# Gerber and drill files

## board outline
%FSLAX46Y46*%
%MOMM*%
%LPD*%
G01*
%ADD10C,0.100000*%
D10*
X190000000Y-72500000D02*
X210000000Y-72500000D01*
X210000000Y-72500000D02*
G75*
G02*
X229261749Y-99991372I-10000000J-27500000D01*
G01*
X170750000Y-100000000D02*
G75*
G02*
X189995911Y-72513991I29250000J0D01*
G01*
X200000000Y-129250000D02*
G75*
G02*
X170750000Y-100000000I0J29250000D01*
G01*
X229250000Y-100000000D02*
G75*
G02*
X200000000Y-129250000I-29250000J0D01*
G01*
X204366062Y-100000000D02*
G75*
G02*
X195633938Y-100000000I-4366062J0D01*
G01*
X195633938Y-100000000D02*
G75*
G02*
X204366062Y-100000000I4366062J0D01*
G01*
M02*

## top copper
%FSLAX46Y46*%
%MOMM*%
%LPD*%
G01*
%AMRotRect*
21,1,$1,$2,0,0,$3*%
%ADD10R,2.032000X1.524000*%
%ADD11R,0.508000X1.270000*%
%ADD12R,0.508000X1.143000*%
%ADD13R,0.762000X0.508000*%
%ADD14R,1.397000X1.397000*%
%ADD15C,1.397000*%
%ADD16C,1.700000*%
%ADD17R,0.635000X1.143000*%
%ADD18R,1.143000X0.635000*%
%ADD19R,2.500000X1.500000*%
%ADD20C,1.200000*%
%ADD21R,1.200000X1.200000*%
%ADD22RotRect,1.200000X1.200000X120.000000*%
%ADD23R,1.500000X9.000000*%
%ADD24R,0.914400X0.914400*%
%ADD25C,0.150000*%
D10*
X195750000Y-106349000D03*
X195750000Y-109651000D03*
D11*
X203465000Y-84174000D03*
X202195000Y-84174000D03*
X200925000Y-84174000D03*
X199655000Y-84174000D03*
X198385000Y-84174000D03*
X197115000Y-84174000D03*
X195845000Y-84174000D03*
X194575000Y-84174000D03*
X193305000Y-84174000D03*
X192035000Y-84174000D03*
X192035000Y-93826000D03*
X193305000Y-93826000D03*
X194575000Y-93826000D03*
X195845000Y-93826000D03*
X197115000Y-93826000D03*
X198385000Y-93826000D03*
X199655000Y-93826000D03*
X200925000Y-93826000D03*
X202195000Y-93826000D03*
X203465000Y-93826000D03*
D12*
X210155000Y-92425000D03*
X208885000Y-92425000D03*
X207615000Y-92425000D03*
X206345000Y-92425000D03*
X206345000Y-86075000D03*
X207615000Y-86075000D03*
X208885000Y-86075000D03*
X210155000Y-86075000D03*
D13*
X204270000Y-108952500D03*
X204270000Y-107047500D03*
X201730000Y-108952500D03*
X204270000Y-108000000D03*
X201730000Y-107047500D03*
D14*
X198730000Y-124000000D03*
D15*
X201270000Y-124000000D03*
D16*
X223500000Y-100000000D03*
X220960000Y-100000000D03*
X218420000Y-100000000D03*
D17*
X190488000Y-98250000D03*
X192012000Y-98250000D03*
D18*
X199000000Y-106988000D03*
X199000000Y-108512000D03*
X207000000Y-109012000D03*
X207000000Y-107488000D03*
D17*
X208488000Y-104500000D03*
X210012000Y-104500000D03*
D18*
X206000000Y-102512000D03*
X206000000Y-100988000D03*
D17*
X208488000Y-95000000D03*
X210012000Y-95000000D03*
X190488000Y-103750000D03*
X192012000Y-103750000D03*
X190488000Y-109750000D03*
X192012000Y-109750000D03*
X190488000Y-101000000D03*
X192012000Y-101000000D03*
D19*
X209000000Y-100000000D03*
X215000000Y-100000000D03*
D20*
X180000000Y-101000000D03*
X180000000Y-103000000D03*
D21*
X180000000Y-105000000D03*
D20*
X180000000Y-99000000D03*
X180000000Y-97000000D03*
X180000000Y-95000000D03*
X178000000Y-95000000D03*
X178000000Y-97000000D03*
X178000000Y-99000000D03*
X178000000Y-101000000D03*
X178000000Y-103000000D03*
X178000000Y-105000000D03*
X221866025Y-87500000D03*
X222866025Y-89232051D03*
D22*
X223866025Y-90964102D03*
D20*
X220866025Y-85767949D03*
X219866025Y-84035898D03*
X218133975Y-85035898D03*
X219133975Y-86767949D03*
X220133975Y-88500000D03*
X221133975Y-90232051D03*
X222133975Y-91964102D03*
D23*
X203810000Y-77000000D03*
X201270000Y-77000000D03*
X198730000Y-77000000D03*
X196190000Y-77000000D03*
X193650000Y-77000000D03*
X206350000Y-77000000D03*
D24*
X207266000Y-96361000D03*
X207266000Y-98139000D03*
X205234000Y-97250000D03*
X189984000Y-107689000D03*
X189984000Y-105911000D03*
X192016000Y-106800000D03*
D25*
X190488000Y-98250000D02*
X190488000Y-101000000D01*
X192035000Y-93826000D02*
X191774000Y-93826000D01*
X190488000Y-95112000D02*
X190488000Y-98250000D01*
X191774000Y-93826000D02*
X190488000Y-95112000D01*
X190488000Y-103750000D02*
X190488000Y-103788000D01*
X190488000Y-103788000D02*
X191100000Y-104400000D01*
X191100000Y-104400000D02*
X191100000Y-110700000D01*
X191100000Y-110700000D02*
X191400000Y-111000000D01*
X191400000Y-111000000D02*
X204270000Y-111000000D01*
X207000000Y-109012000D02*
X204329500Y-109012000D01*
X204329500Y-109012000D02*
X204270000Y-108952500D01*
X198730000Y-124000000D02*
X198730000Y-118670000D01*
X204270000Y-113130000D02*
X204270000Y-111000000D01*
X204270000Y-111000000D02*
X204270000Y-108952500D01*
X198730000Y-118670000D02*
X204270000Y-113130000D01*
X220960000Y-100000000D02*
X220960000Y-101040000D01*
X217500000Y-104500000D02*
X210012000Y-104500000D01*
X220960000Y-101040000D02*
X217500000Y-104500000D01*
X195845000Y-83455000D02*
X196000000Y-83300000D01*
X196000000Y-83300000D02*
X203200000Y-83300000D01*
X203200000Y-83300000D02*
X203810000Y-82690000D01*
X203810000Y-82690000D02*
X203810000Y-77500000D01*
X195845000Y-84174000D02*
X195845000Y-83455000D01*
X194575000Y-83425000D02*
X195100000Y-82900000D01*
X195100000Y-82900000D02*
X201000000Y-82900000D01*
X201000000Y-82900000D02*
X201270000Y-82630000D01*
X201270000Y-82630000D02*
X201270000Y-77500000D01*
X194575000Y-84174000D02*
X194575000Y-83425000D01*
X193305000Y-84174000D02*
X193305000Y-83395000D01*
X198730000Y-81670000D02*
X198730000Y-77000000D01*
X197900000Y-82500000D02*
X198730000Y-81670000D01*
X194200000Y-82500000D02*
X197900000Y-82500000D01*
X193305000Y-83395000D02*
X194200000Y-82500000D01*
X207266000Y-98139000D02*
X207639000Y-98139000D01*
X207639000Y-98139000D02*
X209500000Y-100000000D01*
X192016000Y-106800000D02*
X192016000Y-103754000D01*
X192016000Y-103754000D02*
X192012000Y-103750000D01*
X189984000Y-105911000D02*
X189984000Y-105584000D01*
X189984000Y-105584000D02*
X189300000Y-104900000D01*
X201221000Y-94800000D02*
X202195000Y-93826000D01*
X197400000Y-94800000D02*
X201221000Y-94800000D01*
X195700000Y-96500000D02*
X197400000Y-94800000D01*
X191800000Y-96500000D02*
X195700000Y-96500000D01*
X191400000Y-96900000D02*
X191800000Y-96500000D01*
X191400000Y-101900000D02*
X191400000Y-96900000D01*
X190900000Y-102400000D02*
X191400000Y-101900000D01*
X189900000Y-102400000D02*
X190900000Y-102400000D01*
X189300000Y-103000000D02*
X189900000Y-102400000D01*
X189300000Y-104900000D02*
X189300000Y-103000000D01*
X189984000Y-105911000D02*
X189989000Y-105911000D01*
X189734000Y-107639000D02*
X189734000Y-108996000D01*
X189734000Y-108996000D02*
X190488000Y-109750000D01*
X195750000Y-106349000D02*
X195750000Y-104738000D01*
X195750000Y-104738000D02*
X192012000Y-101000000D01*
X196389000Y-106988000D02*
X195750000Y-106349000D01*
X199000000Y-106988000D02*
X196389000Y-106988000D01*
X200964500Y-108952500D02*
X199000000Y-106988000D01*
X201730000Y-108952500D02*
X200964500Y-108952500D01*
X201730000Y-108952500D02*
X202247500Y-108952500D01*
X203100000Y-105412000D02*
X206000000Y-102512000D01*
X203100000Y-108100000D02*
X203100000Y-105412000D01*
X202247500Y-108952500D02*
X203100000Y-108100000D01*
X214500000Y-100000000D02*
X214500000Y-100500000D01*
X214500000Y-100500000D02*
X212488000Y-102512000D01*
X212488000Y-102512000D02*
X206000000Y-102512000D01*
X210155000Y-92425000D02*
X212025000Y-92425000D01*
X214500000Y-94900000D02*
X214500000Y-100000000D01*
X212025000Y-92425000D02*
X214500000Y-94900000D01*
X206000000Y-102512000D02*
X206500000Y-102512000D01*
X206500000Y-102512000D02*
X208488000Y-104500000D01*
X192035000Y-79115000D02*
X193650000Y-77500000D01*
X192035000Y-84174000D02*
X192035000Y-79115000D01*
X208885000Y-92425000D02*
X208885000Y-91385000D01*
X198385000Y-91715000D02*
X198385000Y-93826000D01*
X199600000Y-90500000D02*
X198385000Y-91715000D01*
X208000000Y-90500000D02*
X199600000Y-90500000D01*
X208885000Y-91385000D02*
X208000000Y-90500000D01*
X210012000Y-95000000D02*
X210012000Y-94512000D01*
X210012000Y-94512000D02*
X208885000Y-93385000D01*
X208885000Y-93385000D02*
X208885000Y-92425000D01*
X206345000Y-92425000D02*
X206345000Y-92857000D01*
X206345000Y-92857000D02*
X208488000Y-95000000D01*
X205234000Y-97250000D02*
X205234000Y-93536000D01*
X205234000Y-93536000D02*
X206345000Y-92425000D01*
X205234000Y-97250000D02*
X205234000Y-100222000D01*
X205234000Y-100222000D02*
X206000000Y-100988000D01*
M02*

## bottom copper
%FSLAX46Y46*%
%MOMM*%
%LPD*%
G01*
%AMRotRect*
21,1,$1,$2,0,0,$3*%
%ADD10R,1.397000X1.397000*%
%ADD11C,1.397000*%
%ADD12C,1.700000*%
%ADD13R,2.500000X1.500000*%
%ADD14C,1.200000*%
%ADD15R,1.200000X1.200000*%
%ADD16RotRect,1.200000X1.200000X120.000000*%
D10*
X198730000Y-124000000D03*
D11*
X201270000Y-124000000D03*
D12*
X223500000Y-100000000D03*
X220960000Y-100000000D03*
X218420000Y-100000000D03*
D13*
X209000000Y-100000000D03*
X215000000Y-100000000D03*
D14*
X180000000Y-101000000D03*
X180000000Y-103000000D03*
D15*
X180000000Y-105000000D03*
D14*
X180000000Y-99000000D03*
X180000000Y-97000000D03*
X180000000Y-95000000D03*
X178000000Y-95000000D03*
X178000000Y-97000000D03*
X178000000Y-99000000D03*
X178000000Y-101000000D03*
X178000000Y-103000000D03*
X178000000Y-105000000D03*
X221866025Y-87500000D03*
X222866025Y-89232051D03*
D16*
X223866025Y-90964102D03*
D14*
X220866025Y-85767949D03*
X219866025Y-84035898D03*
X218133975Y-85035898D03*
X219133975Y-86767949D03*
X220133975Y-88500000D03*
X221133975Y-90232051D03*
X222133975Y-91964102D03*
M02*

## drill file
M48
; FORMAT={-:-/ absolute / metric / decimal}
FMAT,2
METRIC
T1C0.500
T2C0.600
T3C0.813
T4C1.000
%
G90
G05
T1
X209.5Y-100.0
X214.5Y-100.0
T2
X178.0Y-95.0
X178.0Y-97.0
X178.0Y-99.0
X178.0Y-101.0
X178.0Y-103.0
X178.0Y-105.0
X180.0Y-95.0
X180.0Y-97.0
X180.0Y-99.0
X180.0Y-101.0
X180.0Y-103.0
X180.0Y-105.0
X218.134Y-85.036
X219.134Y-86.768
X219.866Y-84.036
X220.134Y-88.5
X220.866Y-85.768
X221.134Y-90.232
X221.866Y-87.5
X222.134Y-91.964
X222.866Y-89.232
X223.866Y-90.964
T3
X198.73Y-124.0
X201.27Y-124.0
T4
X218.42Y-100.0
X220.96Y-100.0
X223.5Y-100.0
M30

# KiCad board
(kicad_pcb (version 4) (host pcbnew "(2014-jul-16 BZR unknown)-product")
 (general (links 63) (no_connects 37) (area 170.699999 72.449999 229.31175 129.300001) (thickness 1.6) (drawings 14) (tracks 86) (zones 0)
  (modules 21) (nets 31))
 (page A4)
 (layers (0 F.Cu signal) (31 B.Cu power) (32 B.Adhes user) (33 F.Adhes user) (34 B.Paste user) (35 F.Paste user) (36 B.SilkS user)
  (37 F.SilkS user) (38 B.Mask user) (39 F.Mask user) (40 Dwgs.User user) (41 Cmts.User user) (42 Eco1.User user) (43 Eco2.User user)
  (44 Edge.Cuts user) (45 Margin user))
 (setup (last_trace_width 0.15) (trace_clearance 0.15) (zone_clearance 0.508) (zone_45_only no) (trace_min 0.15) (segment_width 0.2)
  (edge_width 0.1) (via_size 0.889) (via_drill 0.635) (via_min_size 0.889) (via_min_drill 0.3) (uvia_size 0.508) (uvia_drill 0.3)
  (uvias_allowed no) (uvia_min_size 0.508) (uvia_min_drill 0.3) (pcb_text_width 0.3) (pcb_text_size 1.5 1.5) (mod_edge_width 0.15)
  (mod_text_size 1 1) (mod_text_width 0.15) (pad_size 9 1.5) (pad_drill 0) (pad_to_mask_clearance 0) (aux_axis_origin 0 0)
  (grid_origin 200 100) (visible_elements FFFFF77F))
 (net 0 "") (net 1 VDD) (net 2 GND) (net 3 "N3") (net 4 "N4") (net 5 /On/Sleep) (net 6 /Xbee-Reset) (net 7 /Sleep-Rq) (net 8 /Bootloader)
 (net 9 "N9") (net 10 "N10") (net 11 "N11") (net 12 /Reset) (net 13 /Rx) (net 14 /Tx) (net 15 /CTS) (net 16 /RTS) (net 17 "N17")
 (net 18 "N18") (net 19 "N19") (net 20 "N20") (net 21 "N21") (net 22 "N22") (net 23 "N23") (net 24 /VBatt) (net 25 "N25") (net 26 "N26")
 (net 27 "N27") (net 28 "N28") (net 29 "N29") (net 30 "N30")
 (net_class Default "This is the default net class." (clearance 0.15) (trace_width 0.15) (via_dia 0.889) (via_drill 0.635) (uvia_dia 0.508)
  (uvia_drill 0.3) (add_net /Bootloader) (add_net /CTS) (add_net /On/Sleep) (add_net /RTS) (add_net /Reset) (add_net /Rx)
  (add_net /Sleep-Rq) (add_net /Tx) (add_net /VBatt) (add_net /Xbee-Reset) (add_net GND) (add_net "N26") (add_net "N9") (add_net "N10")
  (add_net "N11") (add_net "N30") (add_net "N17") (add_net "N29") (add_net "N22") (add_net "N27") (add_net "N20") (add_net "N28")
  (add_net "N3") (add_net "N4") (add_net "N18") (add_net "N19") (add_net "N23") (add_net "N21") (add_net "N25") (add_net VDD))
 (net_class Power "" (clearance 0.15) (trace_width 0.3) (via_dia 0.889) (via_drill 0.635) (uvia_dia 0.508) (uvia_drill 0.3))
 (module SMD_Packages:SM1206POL (layer F.Cu) (at 195.75 108 270)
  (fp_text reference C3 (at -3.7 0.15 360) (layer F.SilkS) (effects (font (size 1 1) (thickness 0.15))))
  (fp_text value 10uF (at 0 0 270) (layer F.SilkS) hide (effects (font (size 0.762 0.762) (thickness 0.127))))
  (pad 1 smd rect (at -1.651 0 270) (size 1.524 2.032) (layers F.Cu F.Paste F.Mask) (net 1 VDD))
  (pad 2 smd rect (at 1.651 0 270) (size 1.524 2.032) (layers F.Cu F.Paste F.Mask) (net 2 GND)))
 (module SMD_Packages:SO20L (layer F.Cu) (at 197.75 89)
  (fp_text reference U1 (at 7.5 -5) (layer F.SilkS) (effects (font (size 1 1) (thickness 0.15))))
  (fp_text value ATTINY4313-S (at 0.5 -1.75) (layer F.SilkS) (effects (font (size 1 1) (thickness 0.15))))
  (pad 11 smd rect (at 5.715 -4.826) (size 0.508 1.27) (layers F.Cu F.Paste F.Mask) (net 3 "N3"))
  (pad 12 smd rect (at 4.445 -4.826) (size 0.508 1.27) (layers F.Cu F.Paste F.Mask) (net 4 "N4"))
  (pad 13 smd rect (at 3.175 -4.826) (size 0.508 1.27) (layers F.Cu F.Paste F.Mask) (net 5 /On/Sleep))
  (pad 14 smd rect (at 1.905 -4.826) (size 0.508 1.27) (layers F.Cu F.Paste F.Mask) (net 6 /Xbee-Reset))
  (pad 15 smd rect (at 0.635 -4.826) (size 0.508 1.27) (layers F.Cu F.Paste F.Mask) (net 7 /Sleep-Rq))
  (pad 16 smd rect (at -0.635 -4.826) (size 0.508 1.27) (layers F.Cu F.Paste F.Mask) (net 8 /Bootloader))
  (pad 17 smd rect (at -1.905 -4.826) (size 0.508 1.27) (layers F.Cu F.Paste F.Mask) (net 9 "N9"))
  (pad 18 smd rect (at -3.175 -4.826) (size 0.508 1.27) (layers F.Cu F.Paste F.Mask) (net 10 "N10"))
  (pad 19 smd rect (at -4.445 -4.826) (size 0.508 1.27) (layers F.Cu F.Paste F.Mask) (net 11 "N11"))
  (pad 20 smd rect (at -5.715 -4.826) (size 0.508 1.27) (layers F.Cu F.Paste F.Mask) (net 1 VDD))
  (pad 1 smd rect (at -5.715 4.826) (size 0.508 1.27) (layers F.Cu F.Paste F.Mask) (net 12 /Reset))
  (pad 2 smd rect (at -4.445 4.826) (size 0.508 1.27) (layers F.Cu F.Paste F.Mask) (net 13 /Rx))
  (pad 3 smd rect (at -3.175 4.826) (size 0.508 1.27) (layers F.Cu F.Paste F.Mask) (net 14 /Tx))
  (pad 4 smd rect (at -1.905 4.826) (size 0.508 1.27) (layers F.Cu F.Paste F.Mask) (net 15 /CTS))
  (pad 5 smd rect (at -0.635 4.826) (size 0.508 1.27) (layers F.Cu F.Paste F.Mask) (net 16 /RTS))
  (pad 6 smd rect (at 0.635 4.826) (size 0.508 1.27) (layers F.Cu F.Paste F.Mask) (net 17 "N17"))
  (pad 7 smd rect (at 1.905 4.826) (size 0.508 1.27) (layers F.Cu F.Paste F.Mask) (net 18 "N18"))
  (pad 8 smd rect (at 3.175 4.826) (size 0.508 1.27) (layers F.Cu F.Paste F.Mask) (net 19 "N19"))
  (pad 9 smd rect (at 4.445 4.826) (size 0.508 1.27) (layers F.Cu F.Paste F.Mask) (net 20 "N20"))
  (pad 10 smd rect (at 5.715 4.826) (size 0.508 1.27) (layers F.Cu F.Paste F.Mask) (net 2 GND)))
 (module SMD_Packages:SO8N (layer F.Cu) (at 208.25 89.25 180)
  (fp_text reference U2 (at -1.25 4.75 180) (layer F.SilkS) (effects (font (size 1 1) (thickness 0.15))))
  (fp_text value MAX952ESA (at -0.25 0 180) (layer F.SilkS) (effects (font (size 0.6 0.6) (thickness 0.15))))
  (pad 8 smd rect (at -1.905 -3.175 180) (size 0.508 1.143) (layers F.Cu F.Paste F.Mask) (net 1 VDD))
  (pad 7 smd rect (at -0.635 -3.175 180) (size 0.508 1.143) (layers F.Cu F.Paste F.Mask) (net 17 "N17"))
  (pad 6 smd rect (at 0.635 -3.175 180) (size 0.508 1.143) (layers F.Cu F.Paste F.Mask) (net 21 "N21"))
  (pad 5 smd rect (at 1.905 -3.175 180) (size 0.508 1.143) (layers F.Cu F.Paste F.Mask) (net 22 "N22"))
  (pad 4 smd rect (at 1.905 3.175 180) (size 0.508 1.143) (layers F.Cu F.Paste F.Mask) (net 2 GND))
  (pad 3 smd rect (at 0.635 3.175 180) (size 0.508 1.143) (layers F.Cu F.Paste F.Mask) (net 2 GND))
  (pad 2 smd rect (at -0.635 3.175 180) (size 0.508 1.143) (layers F.Cu F.Paste F.Mask) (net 2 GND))
  (pad 1 smd rect (at -1.905 3.175 180) (size 0.508 1.143) (layers F.Cu F.Paste F.Mask) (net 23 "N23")))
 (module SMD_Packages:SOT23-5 (layer F.Cu) (at 203 108 90)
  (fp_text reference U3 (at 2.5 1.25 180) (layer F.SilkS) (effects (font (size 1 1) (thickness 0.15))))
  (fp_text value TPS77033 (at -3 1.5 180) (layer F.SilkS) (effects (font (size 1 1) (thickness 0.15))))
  (pad 1 smd rect (at -0.9525 1.27 90) (size 0.508 0.762) (layers F.Cu F.Paste F.Mask) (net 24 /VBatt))
  (pad 3 smd rect (at 0.9525 1.27 90) (size 0.508 0.762) (layers F.Cu F.Paste F.Mask) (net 2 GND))
  (pad 5 smd rect (at -0.9525 -1.27 90) (size 0.508 0.762) (layers F.Cu F.Paste F.Mask) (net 1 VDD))
  (pad 2 smd rect (at 0 1.27 90) (size 0.508 0.762) (layers F.Cu F.Paste F.Mask) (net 2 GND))
  (pad 4 smd rect (at 0.9525 -1.27 90) (size 0.508 0.762) (layers F.Cu F.Paste F.Mask) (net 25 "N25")))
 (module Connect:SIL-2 (layer F.Cu) (at 200 124)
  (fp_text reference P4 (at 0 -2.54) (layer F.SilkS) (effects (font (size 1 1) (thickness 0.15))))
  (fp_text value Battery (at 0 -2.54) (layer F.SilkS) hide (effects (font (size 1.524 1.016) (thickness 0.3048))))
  (pad 1 thru_hole rect (at -1.27 0) (size 1.397 1.397) (drill 0.8128) (layers *.Cu *.Mask F.SilkS) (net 24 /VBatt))
  (pad 2 thru_hole circle (at 1.27 0) (size 1.397 1.397) (drill 0.8128) (layers *.Cu *.Mask F.SilkS) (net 2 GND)))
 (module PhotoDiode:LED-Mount (layer F.Cu) (at 223.5 100)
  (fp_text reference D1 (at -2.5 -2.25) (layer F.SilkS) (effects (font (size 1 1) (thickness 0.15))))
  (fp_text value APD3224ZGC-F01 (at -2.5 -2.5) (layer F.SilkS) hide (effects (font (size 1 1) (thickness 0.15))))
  (pad 1 thru_hole circle (at 0 0) (size 1.7 1.7) (drill 1) (layers *.Cu *.Mask F.SilkS) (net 2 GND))
  (pad 2 thru_hole circle (at -2.54 0) (size 1.7 1.7) (drill 1) (layers *.Cu *.Mask F.SilkS) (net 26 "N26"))
  (pad 3 thru_hole circle (at -5.08 0) (size 1.7 1.7) (drill 1) (layers *.Cu *.Mask F.SilkS)))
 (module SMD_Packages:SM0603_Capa (layer F.Cu) (at 191.25 98.25)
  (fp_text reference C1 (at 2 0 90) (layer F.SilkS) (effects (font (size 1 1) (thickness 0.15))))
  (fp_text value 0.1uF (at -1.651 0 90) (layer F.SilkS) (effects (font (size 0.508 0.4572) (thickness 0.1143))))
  (pad 1 smd rect (at -0.762 0) (size 0.635 1.143) (layers F.Cu F.Paste F.Mask) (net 12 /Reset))
  (pad 2 smd rect (at 0.762 0) (size 0.635 1.143) (layers F.Cu F.Paste F.Mask) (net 2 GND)))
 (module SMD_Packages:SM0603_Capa (layer F.Cu) (at 199 107.75 270)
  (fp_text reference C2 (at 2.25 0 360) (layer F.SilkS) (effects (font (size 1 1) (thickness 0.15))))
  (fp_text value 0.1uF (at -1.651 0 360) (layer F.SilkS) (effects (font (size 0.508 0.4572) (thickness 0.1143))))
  (pad 1 smd rect (at -0.762 0 270) (size 0.635 1.143) (layers F.Cu F.Paste F.Mask) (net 1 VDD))
  (pad 2 smd rect (at 0.762 0 270) (size 0.635 1.143) (layers F.Cu F.Paste F.Mask) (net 2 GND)))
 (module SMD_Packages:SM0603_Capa (layer F.Cu) (at 207 108.25 90)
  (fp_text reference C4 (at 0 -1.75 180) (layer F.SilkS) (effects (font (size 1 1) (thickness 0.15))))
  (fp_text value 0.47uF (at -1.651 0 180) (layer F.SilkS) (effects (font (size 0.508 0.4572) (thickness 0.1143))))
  (pad 1 smd rect (at -0.762 0 90) (size 0.635 1.143) (layers F.Cu F.Paste F.Mask) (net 24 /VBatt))
  (pad 2 smd rect (at 0.762 0 90) (size 0.635 1.143) (layers F.Cu F.Paste F.Mask) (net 2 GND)))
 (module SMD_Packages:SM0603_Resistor (layer F.Cu) (at 209.25 104.5)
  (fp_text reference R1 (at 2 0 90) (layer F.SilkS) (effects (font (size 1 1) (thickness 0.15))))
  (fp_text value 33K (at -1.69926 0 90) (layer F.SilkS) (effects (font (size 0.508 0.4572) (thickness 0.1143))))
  (pad 1 smd rect (at -0.762 0) (size 0.635 1.143) (layers F.Cu F.Paste F.Mask) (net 1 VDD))
  (pad 2 smd rect (at 0.762 0) (size 0.635 1.143) (layers F.Cu F.Paste F.Mask) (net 26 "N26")))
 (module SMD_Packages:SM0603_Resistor (layer F.Cu) (at 206 101.75 90)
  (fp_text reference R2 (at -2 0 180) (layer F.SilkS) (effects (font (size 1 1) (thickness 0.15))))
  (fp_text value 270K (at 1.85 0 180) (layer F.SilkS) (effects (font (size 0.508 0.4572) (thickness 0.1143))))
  (pad 1 smd rect (at -0.762 0 90) (size 0.635 1.143) (layers F.Cu F.Paste F.Mask) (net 1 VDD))
  (pad 2 smd rect (at 0.762 0 90) (size 0.635 1.143) (layers F.Cu F.Paste F.Mask) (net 22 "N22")))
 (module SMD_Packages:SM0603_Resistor (layer F.Cu) (at 209.25 95)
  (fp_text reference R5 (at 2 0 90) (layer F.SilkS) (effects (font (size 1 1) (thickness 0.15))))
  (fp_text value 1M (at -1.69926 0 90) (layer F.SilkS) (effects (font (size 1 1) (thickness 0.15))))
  (pad 1 smd rect (at -0.762 0) (size 0.635 1.143) (layers F.Cu F.Paste F.Mask) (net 22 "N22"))
  (pad 2 smd rect (at 0.762 0) (size 0.635 1.143) (layers F.Cu F.Paste F.Mask) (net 17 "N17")))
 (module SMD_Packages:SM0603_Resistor (layer F.Cu) (at 191.25 103.75)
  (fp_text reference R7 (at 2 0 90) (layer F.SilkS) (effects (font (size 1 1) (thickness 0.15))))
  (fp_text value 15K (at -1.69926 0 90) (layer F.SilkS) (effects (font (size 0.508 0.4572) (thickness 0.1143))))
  (pad 1 smd rect (at -0.762 0) (size 0.635 1.143) (layers F.Cu F.Paste F.Mask) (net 24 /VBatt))
  (pad 2 smd rect (at 0.762 0) (size 0.635 1.143) (layers F.Cu F.Paste F.Mask) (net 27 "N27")))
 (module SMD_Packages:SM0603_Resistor (layer F.Cu) (at 191.25 109.75)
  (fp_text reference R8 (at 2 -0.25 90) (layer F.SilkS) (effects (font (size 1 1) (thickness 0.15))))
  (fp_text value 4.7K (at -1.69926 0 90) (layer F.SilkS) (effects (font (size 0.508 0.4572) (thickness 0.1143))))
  (pad 1 smd rect (at -0.762 0) (size 0.635 1.143) (layers F.Cu F.Paste F.Mask) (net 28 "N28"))
  (pad 2 smd rect (at 0.762 0) (size 0.635 1.143) (layers F.Cu F.Paste F.Mask) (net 2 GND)))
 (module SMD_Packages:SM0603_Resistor (layer F.Cu) (at 191.25 101)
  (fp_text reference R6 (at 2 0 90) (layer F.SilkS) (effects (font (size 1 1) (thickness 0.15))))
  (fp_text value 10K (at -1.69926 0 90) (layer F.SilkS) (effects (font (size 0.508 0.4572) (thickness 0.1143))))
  (pad 1 smd rect (at -0.762 0) (size 0.635 1.143) (layers F.Cu F.Paste F.Mask) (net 12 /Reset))
  (pad 2 smd rect (at 0.762 0) (size 0.635 1.143) (layers F.Cu F.Paste F.Mask) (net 1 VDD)))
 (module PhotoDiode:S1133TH (layer F.Cu) (at 212 100)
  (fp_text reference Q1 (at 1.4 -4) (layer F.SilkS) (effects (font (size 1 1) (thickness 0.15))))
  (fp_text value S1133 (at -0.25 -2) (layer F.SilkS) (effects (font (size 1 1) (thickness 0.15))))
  (pad 1 thru_hole rect (at -2.5 0) (size 2.5 1.5) (drill 0.5 (offset -0.5 0)) (layers *.Cu *.Mask F.SilkS) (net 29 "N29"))
  (pad 3 thru_hole rect (at 2.5 0) (size 2.5 1.5) (drill 0.5 (offset 0.5 0)) (layers *.Cu *.Mask F.SilkS) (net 1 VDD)))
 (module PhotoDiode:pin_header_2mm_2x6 (layer F.Cu) (at 179 100 90)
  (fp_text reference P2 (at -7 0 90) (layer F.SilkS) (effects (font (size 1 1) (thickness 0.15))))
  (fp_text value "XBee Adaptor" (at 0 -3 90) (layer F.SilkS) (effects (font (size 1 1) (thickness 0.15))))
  (pad 5 thru_hole circle (at -1 1 90) (size 1.2 1.2) (drill 0.6) (layers *.Cu *.Mask F.SilkS) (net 14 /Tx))
  (pad 3 thru_hole circle (at -3 1 90) (size 1.2 1.2) (drill 0.6) (layers *.Cu *.Mask F.SilkS) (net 13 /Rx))
  (pad 1 thru_hole rect (at -5 1 90) (size 1.2 1.2) (drill 0.6) (layers *.Cu *.Mask F.SilkS) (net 1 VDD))
  (pad 7 thru_hole circle (at 1 1 90) (size 1.2 1.2) (drill 0.6) (layers *.Cu *.Mask F.SilkS) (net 8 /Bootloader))
  (pad 9 thru_hole circle (at 3 1 90) (size 1.2 1.2) (drill 0.6) (layers *.Cu *.Mask F.SilkS) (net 12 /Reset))
  (pad 11 thru_hole circle (at 5 1 90) (size 1.2 1.2) (drill 0.6) (layers *.Cu *.Mask F.SilkS) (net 2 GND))
  (pad 12 thru_hole circle (at 5 -1 90) (size 1.2 1.2) (drill 0.6) (layers *.Cu *.Mask F.SilkS) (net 24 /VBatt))
  (pad 10 thru_hole circle (at 3 -1 90) (size 1.2 1.2) (drill 0.6) (layers *.Cu *.Mask F.SilkS) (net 6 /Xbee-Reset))
  (pad 8 thru_hole circle (at 1 -1 90) (size 1.2 1.2) (drill 0.6) (layers *.Cu *.Mask F.SilkS) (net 5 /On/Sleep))
  (pad 6 thru_hole circle (at -1 -1 90) (size 1.2 1.2) (drill 0.6) (layers *.Cu *.Mask F.SilkS) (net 16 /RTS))
  (pad 4 thru_hole circle (at -3 -1 90) (size 1.2 1.2) (drill 0.6) (layers *.Cu *.Mask F.SilkS) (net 15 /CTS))
  (pad 2 thru_hole circle (at -5 -1 90) (size 1.2 1.2) (drill 0.6) (layers *.Cu *.Mask F.SilkS) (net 7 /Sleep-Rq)))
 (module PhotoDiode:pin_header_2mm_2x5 (layer F.Cu) (at 221 88 120)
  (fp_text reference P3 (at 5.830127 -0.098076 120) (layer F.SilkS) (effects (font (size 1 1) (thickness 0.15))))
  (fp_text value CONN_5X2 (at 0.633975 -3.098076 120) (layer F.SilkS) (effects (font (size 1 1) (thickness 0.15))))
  (pad 5 thru_hole circle (at 0 1 120) (size 1.2 1.2) (drill 0.6) (layers *.Cu *.Mask F.SilkS) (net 17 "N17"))
  (pad 3 thru_hole circle (at -2 1 120) (size 1.2 1.2) (drill 0.6) (layers *.Cu *.Mask F.SilkS) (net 14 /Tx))
  (pad 1 thru_hole rect (at -4 1 120) (size 1.2 1.2) (drill 0.6) (layers *.Cu *.Mask F.SilkS) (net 13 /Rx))
  (pad 7 thru_hole circle (at 2 1 120) (size 1.2 1.2) (drill 0.6) (layers *.Cu *.Mask F.SilkS) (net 12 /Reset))
  (pad 9 thru_hole circle (at 4 1 120) (size 1.2 1.2) (drill 0.6) (layers *.Cu *.Mask F.SilkS) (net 2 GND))
  (pad 10 thru_hole circle (at 4 -1 120) (size 1.2 1.2) (drill 0.6) (layers *.Cu *.Mask F.SilkS) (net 24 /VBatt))
  (pad 8 thru_hole circle (at 2 -1 120) (size 1.2 1.2) (drill 0.6) (layers *.Cu *.Mask F.SilkS) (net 6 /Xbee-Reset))
  (pad 6 thru_hole circle (at 0 -1 120) (size 1.2 1.2) (drill 0.6) (layers *.Cu *.Mask F.SilkS) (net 5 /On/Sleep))
  (pad 4 thru_hole circle (at -2 -1 120) (size 1.2 1.2) (drill 0.6) (layers *.Cu *.Mask F.SilkS) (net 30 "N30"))
  (pad 2 thru_hole circle (at -4 -1 120) (size 1.2 1.2) (drill 0.6) (layers *.Cu *.Mask F.SilkS) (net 7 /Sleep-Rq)))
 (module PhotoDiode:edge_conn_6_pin (layer F.Cu) (at 200 77 90)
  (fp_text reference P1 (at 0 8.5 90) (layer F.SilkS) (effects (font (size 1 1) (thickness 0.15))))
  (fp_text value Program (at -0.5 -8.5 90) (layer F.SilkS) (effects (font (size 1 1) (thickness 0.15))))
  (pad 2 connect rect (at 0 3.81 90) (size 9 1.5) (layers F.Cu F.Mask) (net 9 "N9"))
  (pad 3 connect rect (at 0 1.27 90) (size 9 1.5) (layers F.Cu F.Mask) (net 10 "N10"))
  (pad 4 connect rect (at 0 -1.27 90) (size 9 1.5) (layers F.Cu F.Mask) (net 11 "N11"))
  (pad 5 connect rect (at 0 -3.81 90) (size 9 1.5) (layers F.Cu F.Mask) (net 12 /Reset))
  (pad 6 connect rect (at 0 -6.35 90) (size 9 1.5) (layers F.Cu F.Mask) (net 1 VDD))
  (pad 1 connect rect (at 0 6.35 90) (size 9 1.5) (layers F.Cu F.Mask) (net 2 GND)))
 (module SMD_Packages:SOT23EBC (layer F.Cu) (at 206.25 97.25 270)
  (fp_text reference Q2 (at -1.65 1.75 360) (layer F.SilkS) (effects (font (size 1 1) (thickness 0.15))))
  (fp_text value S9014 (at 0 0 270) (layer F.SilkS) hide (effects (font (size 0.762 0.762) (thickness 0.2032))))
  (pad 1 smd rect (at -0.889 -1.016 270) (size 0.9144 0.9144) (layers F.Cu F.Paste F.Mask) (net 2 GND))
  (pad 2 smd rect (at 0.889 -1.016 270) (size 0.9144 0.9144) (layers F.Cu F.Paste F.Mask) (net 29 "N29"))
  (pad 3 smd rect (at 0 1.016 270) (size 0.9144 0.9144) (layers F.Cu F.Paste F.Mask) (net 22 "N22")))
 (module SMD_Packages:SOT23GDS (layer F.Cu) (at 191 106.8 90)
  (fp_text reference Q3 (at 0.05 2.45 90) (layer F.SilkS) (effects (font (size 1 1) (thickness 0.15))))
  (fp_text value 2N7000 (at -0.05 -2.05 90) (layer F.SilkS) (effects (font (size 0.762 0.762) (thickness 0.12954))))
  (pad S smd rect (at -0.889 -1.016 90) (size 0.9144 0.9144) (layers F.Cu F.Paste F.Mask) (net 28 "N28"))
  (pad G smd rect (at 0.889 -1.016 90) (size 0.9144 0.9144) (layers F.Cu F.Paste F.Mask) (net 20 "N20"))
  (pad D smd rect (at 0 1.016 90) (size 0.9144 0.9144) (layers F.Cu F.Paste F.Mask) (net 27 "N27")))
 (gr_line (start 190 72.5) (end 210 72.5) (angle 90) (layer Edge.Cuts) (width 0.1))
 (gr_arc (start 200 100) (end 210 72.5) (angle 70) (layer Edge.Cuts) (width 0.1))
 (gr_arc (start 200 100) (end 170.75 100) (angle 70) (layer Edge.Cuts) (width 0.1))
 (gr_arc (start 200 100) (end 200 129.25) (angle 90) (layer Edge.Cuts) (width 0.1))
 (gr_arc (start 200 100) (end 229.25 100) (angle 90) (layer Edge.Cuts) (width 0.1))
 (gr_circle (center 200 100) (end 204.25 101) (layer Edge.Cuts) (width 0.1))
 (segment (start 190.488 98.25) (end 190.488 101) (width 0.15) (layer F.Cu) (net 12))
 (segment (start 192.035 93.826) (end 191.774 93.826) (width 0.15) (layer F.Cu) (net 12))
 (segment (start 190.488 95.112) (end 190.488 98.25) (width 0.15) (layer F.Cu) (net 12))
 (segment (start 191.774 93.826) (end 190.488 95.112) (width 0.15) (layer F.Cu) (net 12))
 (segment (start 190.488 103.75) (end 190.488 103.788) (width 0.15) (layer F.Cu) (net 24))
 (segment (start 190.488 103.788) (end 191.1 104.4) (width 0.15) (layer F.Cu) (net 24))
 (segment (start 191.1 104.4) (end 191.1 110.7) (width 0.15) (layer F.Cu) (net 24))
 (segment (start 191.1 110.7) (end 191.4 111) (width 0.15) (layer F.Cu) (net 24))
 (segment (start 191.4 111) (end 204.27 111) (width 0.15) (layer F.Cu) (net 24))
 (segment (start 207 109.012) (end 204.3295 109.012) (width 0.15) (layer F.Cu) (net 24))
 (segment (start 204.3295 109.012) (end 204.27 108.9525) (width 0.15) (layer F.Cu) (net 24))
 (segment (start 198.73 124) (end 198.73 118.67) (width 0.15) (layer F.Cu) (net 24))
 (segment (start 204.27 113.13) (end 204.27 111) (width 0.15) (layer F.Cu) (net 24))
 (segment (start 204.27 111) (end 204.27 108.9525) (width 0.15) (layer F.Cu) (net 24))
 (segment (start 198.73 118.67) (end 204.27 113.13) (width 0.15) (layer F.Cu) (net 24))
 (segment (start 220.96 100) (end 220.96 101.04) (width 0.15) (layer F.Cu) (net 26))
 (segment (start 217.5 104.5) (end 210.012 104.5) (width 0.15) (layer F.Cu) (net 26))
 (segment (start 220.96 101.04) (end 217.5 104.5) (width 0.15) (layer F.Cu) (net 26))
 (segment (start 195.845 83.455) (end 196 83.3) (width 0.15) (layer F.Cu) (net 9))
 (segment (start 196 83.3) (end 203.2 83.3) (width 0.15) (layer F.Cu) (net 9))
 (segment (start 203.2 83.3) (end 203.81 82.69) (width 0.15) (layer F.Cu) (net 9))
 (segment (start 203.81 82.69) (end 203.81 77.5) (width 0.15) (layer F.Cu) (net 9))
 (segment (start 195.845 84.174) (end 195.845 83.455) (width 0.15) (layer F.Cu) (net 9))
 (segment (start 194.575 83.425) (end 195.1 82.9) (width 0.15) (layer F.Cu) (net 10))
 (segment (start 195.1 82.9) (end 201 82.9) (width 0.15) (layer F.Cu) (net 10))
 (segment (start 201 82.9) (end 201.27 82.63) (width 0.15) (layer F.Cu) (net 10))
 (segment (start 201.27 82.63) (end 201.27 77.5) (width 0.15) (layer F.Cu) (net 10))
 (segment (start 194.575 84.174) (end 194.575 83.425) (width 0.15) (layer F.Cu) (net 10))
 (segment (start 193.305 84.174) (end 193.305 83.395) (width 0.15) (layer F.Cu) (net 11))
 (segment (start 198.73 81.67) (end 198.73 77) (width 0.15) (layer F.Cu) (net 11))
 (segment (start 197.9 82.5) (end 198.73 81.67) (width 0.15) (layer F.Cu) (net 11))
 (segment (start 194.2 82.5) (end 197.9 82.5) (width 0.15) (layer F.Cu) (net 11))
 (segment (start 193.305 83.395) (end 194.2 82.5) (width 0.15) (layer F.Cu) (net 11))
 (segment (start 207.266 98.139) (end 207.639 98.139) (width 0.15) (layer F.Cu) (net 29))
 (segment (start 207.639 98.139) (end 209.5 100) (width 0.15) (layer F.Cu) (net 29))
 (segment (start 192.016 106.8) (end 192.016 103.754) (width 0.15) (layer F.Cu) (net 27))
 (segment (start 192.016 103.754) (end 192.012 103.75) (width 0.15) (layer F.Cu) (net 27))
 (segment (start 189.984 105.911) (end 189.984 105.584) (width 0.15) (layer F.Cu) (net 20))
 (segment (start 189.984 105.584) (end 189.3 104.9) (width 0.15) (layer F.Cu) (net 20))
 (segment (start 201.221 94.8) (end 202.195 93.826) (width 0.15) (layer F.Cu) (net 20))
 (segment (start 197.4 94.8) (end 201.221 94.8) (width 0.15) (layer F.Cu) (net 20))
 (segment (start 195.7 96.5) (end 197.4 94.8) (width 0.15) (layer F.Cu) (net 20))
 (segment (start 191.8 96.5) (end 195.7 96.5) (width 0.15) (layer F.Cu) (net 20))
 (segment (start 191.4 96.9) (end 191.8 96.5) (width 0.15) (layer F.Cu) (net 20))
 (segment (start 191.4 101.9) (end 191.4 96.9) (width 0.15) (layer F.Cu) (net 20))
 (segment (start 190.9 102.4) (end 191.4 101.9) (width 0.15) (layer F.Cu) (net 20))
 (segment (start 189.9 102.4) (end 190.9 102.4) (width 0.15) (layer F.Cu) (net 20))
 (segment (start 189.3 103) (end 189.9 102.4) (width 0.15) (layer F.Cu) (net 20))
 (segment (start 189.3 104.9) (end 189.3 103) (width 0.15) (layer F.Cu) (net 20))
 (segment (start 189.984 105.911) (end 189.989 105.911) (width 0.15) (layer F.Cu) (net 20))
 (segment (start 189.734 107.639) (end 189.734 108.996) (width 0.15) (layer F.Cu) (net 28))
 (segment (start 189.734 108.996) (end 190.488 109.75) (width 0.15) (layer F.Cu) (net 28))
 (segment (start 195.75 106.349) (end 195.75 104.738) (width 0.15) (layer F.Cu) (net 1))
 (segment (start 195.75 104.738) (end 192.012 101) (width 0.15) (layer F.Cu) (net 1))
 (segment (start 196.389 106.988) (end 195.75 106.349) (width 0.15) (layer F.Cu) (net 1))
 (segment (start 199 106.988) (end 196.389 106.988) (width 0.15) (layer F.Cu) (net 1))
 (segment (start 200.9645 108.9525) (end 199 106.988) (width 0.15) (layer F.Cu) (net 1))
 (segment (start 201.73 108.9525) (end 200.9645 108.9525) (width 0.15) (layer F.Cu) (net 1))
 (segment (start 201.73 108.9525) (end 202.2475 108.9525) (width 0.15) (layer F.Cu) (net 1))
 (segment (start 203.1 105.412) (end 206 102.512) (width 0.15) (layer F.Cu) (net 1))
 (segment (start 203.1 108.1) (end 203.1 105.412) (width 0.15) (layer F.Cu) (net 1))
 (segment (start 202.2475 108.9525) (end 203.1 108.1) (width 0.15) (layer F.Cu) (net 1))
 (segment (start 214.5 100) (end 214.5 100.5) (width 0.15) (layer F.Cu) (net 1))
 (segment (start 214.5 100.5) (end 212.488 102.512) (width 0.15) (layer F.Cu) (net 1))
 (segment (start 212.488 102.512) (end 206 102.512) (width 0.15) (layer F.Cu) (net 1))
 (segment (start 210.155 92.425) (end 212.025 92.425) (width 0.15) (layer F.Cu) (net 1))
 (segment (start 214.5 94.9) (end 214.5 100) (width 0.15) (layer F.Cu) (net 1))
 (segment (start 212.025 92.425) (end 214.5 94.9) (width 0.15) (layer F.Cu) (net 1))
 (segment (start 206 102.512) (end 206.5 102.512) (width 0.15) (layer F.Cu) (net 1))
 (segment (start 206.5 102.512) (end 208.488 104.5) (width 0.15) (layer F.Cu) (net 1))
 (segment (start 192.035 79.115) (end 193.65 77.5) (width 0.15) (layer F.Cu) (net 1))
 (segment (start 192.035 84.174) (end 192.035 79.115) (width 0.15) (layer F.Cu) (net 1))
 (segment (start 208.885 92.425) (end 208.885 91.385) (width 0.15) (layer F.Cu) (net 17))
 (segment (start 198.385 91.715) (end 198.385 93.826) (width 0.15) (layer F.Cu) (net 17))
 (segment (start 199.6 90.5) (end 198.385 91.715) (width 0.15) (layer F.Cu) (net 17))
 (segment (start 208 90.5) (end 199.6 90.5) (width 0.15) (layer F.Cu) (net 17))
 (segment (start 208.885 91.385) (end 208 90.5) (width 0.15) (layer F.Cu) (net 17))
 (segment (start 210.012 95) (end 210.012 94.512) (width 0.15) (layer F.Cu) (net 17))
 (segment (start 210.012 94.512) (end 208.885 93.385) (width 0.15) (layer F.Cu) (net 17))
 (segment (start 208.885 93.385) (end 208.885 92.425) (width 0.15) (layer F.Cu) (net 17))
 (segment (start 206.345 92.425) (end 206.345 92.857) (width 0.15) (layer F.Cu) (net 22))
 (segment (start 206.345 92.857) (end 208.488 95) (width 0.15) (layer F.Cu) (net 22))
 (segment (start 205.234 97.25) (end 205.234 93.536) (width 0.15) (layer F.Cu) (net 22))
 (segment (start 205.234 93.536) (end 206.345 92.425) (width 0.15) (layer F.Cu) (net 22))
 (segment (start 205.234 97.25) (end 205.234 100.222) (width 0.15) (layer F.Cu) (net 22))
 (segment (start 205.234 100.222) (end 206 100.988) (width 0.15) (layer F.Cu) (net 22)))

